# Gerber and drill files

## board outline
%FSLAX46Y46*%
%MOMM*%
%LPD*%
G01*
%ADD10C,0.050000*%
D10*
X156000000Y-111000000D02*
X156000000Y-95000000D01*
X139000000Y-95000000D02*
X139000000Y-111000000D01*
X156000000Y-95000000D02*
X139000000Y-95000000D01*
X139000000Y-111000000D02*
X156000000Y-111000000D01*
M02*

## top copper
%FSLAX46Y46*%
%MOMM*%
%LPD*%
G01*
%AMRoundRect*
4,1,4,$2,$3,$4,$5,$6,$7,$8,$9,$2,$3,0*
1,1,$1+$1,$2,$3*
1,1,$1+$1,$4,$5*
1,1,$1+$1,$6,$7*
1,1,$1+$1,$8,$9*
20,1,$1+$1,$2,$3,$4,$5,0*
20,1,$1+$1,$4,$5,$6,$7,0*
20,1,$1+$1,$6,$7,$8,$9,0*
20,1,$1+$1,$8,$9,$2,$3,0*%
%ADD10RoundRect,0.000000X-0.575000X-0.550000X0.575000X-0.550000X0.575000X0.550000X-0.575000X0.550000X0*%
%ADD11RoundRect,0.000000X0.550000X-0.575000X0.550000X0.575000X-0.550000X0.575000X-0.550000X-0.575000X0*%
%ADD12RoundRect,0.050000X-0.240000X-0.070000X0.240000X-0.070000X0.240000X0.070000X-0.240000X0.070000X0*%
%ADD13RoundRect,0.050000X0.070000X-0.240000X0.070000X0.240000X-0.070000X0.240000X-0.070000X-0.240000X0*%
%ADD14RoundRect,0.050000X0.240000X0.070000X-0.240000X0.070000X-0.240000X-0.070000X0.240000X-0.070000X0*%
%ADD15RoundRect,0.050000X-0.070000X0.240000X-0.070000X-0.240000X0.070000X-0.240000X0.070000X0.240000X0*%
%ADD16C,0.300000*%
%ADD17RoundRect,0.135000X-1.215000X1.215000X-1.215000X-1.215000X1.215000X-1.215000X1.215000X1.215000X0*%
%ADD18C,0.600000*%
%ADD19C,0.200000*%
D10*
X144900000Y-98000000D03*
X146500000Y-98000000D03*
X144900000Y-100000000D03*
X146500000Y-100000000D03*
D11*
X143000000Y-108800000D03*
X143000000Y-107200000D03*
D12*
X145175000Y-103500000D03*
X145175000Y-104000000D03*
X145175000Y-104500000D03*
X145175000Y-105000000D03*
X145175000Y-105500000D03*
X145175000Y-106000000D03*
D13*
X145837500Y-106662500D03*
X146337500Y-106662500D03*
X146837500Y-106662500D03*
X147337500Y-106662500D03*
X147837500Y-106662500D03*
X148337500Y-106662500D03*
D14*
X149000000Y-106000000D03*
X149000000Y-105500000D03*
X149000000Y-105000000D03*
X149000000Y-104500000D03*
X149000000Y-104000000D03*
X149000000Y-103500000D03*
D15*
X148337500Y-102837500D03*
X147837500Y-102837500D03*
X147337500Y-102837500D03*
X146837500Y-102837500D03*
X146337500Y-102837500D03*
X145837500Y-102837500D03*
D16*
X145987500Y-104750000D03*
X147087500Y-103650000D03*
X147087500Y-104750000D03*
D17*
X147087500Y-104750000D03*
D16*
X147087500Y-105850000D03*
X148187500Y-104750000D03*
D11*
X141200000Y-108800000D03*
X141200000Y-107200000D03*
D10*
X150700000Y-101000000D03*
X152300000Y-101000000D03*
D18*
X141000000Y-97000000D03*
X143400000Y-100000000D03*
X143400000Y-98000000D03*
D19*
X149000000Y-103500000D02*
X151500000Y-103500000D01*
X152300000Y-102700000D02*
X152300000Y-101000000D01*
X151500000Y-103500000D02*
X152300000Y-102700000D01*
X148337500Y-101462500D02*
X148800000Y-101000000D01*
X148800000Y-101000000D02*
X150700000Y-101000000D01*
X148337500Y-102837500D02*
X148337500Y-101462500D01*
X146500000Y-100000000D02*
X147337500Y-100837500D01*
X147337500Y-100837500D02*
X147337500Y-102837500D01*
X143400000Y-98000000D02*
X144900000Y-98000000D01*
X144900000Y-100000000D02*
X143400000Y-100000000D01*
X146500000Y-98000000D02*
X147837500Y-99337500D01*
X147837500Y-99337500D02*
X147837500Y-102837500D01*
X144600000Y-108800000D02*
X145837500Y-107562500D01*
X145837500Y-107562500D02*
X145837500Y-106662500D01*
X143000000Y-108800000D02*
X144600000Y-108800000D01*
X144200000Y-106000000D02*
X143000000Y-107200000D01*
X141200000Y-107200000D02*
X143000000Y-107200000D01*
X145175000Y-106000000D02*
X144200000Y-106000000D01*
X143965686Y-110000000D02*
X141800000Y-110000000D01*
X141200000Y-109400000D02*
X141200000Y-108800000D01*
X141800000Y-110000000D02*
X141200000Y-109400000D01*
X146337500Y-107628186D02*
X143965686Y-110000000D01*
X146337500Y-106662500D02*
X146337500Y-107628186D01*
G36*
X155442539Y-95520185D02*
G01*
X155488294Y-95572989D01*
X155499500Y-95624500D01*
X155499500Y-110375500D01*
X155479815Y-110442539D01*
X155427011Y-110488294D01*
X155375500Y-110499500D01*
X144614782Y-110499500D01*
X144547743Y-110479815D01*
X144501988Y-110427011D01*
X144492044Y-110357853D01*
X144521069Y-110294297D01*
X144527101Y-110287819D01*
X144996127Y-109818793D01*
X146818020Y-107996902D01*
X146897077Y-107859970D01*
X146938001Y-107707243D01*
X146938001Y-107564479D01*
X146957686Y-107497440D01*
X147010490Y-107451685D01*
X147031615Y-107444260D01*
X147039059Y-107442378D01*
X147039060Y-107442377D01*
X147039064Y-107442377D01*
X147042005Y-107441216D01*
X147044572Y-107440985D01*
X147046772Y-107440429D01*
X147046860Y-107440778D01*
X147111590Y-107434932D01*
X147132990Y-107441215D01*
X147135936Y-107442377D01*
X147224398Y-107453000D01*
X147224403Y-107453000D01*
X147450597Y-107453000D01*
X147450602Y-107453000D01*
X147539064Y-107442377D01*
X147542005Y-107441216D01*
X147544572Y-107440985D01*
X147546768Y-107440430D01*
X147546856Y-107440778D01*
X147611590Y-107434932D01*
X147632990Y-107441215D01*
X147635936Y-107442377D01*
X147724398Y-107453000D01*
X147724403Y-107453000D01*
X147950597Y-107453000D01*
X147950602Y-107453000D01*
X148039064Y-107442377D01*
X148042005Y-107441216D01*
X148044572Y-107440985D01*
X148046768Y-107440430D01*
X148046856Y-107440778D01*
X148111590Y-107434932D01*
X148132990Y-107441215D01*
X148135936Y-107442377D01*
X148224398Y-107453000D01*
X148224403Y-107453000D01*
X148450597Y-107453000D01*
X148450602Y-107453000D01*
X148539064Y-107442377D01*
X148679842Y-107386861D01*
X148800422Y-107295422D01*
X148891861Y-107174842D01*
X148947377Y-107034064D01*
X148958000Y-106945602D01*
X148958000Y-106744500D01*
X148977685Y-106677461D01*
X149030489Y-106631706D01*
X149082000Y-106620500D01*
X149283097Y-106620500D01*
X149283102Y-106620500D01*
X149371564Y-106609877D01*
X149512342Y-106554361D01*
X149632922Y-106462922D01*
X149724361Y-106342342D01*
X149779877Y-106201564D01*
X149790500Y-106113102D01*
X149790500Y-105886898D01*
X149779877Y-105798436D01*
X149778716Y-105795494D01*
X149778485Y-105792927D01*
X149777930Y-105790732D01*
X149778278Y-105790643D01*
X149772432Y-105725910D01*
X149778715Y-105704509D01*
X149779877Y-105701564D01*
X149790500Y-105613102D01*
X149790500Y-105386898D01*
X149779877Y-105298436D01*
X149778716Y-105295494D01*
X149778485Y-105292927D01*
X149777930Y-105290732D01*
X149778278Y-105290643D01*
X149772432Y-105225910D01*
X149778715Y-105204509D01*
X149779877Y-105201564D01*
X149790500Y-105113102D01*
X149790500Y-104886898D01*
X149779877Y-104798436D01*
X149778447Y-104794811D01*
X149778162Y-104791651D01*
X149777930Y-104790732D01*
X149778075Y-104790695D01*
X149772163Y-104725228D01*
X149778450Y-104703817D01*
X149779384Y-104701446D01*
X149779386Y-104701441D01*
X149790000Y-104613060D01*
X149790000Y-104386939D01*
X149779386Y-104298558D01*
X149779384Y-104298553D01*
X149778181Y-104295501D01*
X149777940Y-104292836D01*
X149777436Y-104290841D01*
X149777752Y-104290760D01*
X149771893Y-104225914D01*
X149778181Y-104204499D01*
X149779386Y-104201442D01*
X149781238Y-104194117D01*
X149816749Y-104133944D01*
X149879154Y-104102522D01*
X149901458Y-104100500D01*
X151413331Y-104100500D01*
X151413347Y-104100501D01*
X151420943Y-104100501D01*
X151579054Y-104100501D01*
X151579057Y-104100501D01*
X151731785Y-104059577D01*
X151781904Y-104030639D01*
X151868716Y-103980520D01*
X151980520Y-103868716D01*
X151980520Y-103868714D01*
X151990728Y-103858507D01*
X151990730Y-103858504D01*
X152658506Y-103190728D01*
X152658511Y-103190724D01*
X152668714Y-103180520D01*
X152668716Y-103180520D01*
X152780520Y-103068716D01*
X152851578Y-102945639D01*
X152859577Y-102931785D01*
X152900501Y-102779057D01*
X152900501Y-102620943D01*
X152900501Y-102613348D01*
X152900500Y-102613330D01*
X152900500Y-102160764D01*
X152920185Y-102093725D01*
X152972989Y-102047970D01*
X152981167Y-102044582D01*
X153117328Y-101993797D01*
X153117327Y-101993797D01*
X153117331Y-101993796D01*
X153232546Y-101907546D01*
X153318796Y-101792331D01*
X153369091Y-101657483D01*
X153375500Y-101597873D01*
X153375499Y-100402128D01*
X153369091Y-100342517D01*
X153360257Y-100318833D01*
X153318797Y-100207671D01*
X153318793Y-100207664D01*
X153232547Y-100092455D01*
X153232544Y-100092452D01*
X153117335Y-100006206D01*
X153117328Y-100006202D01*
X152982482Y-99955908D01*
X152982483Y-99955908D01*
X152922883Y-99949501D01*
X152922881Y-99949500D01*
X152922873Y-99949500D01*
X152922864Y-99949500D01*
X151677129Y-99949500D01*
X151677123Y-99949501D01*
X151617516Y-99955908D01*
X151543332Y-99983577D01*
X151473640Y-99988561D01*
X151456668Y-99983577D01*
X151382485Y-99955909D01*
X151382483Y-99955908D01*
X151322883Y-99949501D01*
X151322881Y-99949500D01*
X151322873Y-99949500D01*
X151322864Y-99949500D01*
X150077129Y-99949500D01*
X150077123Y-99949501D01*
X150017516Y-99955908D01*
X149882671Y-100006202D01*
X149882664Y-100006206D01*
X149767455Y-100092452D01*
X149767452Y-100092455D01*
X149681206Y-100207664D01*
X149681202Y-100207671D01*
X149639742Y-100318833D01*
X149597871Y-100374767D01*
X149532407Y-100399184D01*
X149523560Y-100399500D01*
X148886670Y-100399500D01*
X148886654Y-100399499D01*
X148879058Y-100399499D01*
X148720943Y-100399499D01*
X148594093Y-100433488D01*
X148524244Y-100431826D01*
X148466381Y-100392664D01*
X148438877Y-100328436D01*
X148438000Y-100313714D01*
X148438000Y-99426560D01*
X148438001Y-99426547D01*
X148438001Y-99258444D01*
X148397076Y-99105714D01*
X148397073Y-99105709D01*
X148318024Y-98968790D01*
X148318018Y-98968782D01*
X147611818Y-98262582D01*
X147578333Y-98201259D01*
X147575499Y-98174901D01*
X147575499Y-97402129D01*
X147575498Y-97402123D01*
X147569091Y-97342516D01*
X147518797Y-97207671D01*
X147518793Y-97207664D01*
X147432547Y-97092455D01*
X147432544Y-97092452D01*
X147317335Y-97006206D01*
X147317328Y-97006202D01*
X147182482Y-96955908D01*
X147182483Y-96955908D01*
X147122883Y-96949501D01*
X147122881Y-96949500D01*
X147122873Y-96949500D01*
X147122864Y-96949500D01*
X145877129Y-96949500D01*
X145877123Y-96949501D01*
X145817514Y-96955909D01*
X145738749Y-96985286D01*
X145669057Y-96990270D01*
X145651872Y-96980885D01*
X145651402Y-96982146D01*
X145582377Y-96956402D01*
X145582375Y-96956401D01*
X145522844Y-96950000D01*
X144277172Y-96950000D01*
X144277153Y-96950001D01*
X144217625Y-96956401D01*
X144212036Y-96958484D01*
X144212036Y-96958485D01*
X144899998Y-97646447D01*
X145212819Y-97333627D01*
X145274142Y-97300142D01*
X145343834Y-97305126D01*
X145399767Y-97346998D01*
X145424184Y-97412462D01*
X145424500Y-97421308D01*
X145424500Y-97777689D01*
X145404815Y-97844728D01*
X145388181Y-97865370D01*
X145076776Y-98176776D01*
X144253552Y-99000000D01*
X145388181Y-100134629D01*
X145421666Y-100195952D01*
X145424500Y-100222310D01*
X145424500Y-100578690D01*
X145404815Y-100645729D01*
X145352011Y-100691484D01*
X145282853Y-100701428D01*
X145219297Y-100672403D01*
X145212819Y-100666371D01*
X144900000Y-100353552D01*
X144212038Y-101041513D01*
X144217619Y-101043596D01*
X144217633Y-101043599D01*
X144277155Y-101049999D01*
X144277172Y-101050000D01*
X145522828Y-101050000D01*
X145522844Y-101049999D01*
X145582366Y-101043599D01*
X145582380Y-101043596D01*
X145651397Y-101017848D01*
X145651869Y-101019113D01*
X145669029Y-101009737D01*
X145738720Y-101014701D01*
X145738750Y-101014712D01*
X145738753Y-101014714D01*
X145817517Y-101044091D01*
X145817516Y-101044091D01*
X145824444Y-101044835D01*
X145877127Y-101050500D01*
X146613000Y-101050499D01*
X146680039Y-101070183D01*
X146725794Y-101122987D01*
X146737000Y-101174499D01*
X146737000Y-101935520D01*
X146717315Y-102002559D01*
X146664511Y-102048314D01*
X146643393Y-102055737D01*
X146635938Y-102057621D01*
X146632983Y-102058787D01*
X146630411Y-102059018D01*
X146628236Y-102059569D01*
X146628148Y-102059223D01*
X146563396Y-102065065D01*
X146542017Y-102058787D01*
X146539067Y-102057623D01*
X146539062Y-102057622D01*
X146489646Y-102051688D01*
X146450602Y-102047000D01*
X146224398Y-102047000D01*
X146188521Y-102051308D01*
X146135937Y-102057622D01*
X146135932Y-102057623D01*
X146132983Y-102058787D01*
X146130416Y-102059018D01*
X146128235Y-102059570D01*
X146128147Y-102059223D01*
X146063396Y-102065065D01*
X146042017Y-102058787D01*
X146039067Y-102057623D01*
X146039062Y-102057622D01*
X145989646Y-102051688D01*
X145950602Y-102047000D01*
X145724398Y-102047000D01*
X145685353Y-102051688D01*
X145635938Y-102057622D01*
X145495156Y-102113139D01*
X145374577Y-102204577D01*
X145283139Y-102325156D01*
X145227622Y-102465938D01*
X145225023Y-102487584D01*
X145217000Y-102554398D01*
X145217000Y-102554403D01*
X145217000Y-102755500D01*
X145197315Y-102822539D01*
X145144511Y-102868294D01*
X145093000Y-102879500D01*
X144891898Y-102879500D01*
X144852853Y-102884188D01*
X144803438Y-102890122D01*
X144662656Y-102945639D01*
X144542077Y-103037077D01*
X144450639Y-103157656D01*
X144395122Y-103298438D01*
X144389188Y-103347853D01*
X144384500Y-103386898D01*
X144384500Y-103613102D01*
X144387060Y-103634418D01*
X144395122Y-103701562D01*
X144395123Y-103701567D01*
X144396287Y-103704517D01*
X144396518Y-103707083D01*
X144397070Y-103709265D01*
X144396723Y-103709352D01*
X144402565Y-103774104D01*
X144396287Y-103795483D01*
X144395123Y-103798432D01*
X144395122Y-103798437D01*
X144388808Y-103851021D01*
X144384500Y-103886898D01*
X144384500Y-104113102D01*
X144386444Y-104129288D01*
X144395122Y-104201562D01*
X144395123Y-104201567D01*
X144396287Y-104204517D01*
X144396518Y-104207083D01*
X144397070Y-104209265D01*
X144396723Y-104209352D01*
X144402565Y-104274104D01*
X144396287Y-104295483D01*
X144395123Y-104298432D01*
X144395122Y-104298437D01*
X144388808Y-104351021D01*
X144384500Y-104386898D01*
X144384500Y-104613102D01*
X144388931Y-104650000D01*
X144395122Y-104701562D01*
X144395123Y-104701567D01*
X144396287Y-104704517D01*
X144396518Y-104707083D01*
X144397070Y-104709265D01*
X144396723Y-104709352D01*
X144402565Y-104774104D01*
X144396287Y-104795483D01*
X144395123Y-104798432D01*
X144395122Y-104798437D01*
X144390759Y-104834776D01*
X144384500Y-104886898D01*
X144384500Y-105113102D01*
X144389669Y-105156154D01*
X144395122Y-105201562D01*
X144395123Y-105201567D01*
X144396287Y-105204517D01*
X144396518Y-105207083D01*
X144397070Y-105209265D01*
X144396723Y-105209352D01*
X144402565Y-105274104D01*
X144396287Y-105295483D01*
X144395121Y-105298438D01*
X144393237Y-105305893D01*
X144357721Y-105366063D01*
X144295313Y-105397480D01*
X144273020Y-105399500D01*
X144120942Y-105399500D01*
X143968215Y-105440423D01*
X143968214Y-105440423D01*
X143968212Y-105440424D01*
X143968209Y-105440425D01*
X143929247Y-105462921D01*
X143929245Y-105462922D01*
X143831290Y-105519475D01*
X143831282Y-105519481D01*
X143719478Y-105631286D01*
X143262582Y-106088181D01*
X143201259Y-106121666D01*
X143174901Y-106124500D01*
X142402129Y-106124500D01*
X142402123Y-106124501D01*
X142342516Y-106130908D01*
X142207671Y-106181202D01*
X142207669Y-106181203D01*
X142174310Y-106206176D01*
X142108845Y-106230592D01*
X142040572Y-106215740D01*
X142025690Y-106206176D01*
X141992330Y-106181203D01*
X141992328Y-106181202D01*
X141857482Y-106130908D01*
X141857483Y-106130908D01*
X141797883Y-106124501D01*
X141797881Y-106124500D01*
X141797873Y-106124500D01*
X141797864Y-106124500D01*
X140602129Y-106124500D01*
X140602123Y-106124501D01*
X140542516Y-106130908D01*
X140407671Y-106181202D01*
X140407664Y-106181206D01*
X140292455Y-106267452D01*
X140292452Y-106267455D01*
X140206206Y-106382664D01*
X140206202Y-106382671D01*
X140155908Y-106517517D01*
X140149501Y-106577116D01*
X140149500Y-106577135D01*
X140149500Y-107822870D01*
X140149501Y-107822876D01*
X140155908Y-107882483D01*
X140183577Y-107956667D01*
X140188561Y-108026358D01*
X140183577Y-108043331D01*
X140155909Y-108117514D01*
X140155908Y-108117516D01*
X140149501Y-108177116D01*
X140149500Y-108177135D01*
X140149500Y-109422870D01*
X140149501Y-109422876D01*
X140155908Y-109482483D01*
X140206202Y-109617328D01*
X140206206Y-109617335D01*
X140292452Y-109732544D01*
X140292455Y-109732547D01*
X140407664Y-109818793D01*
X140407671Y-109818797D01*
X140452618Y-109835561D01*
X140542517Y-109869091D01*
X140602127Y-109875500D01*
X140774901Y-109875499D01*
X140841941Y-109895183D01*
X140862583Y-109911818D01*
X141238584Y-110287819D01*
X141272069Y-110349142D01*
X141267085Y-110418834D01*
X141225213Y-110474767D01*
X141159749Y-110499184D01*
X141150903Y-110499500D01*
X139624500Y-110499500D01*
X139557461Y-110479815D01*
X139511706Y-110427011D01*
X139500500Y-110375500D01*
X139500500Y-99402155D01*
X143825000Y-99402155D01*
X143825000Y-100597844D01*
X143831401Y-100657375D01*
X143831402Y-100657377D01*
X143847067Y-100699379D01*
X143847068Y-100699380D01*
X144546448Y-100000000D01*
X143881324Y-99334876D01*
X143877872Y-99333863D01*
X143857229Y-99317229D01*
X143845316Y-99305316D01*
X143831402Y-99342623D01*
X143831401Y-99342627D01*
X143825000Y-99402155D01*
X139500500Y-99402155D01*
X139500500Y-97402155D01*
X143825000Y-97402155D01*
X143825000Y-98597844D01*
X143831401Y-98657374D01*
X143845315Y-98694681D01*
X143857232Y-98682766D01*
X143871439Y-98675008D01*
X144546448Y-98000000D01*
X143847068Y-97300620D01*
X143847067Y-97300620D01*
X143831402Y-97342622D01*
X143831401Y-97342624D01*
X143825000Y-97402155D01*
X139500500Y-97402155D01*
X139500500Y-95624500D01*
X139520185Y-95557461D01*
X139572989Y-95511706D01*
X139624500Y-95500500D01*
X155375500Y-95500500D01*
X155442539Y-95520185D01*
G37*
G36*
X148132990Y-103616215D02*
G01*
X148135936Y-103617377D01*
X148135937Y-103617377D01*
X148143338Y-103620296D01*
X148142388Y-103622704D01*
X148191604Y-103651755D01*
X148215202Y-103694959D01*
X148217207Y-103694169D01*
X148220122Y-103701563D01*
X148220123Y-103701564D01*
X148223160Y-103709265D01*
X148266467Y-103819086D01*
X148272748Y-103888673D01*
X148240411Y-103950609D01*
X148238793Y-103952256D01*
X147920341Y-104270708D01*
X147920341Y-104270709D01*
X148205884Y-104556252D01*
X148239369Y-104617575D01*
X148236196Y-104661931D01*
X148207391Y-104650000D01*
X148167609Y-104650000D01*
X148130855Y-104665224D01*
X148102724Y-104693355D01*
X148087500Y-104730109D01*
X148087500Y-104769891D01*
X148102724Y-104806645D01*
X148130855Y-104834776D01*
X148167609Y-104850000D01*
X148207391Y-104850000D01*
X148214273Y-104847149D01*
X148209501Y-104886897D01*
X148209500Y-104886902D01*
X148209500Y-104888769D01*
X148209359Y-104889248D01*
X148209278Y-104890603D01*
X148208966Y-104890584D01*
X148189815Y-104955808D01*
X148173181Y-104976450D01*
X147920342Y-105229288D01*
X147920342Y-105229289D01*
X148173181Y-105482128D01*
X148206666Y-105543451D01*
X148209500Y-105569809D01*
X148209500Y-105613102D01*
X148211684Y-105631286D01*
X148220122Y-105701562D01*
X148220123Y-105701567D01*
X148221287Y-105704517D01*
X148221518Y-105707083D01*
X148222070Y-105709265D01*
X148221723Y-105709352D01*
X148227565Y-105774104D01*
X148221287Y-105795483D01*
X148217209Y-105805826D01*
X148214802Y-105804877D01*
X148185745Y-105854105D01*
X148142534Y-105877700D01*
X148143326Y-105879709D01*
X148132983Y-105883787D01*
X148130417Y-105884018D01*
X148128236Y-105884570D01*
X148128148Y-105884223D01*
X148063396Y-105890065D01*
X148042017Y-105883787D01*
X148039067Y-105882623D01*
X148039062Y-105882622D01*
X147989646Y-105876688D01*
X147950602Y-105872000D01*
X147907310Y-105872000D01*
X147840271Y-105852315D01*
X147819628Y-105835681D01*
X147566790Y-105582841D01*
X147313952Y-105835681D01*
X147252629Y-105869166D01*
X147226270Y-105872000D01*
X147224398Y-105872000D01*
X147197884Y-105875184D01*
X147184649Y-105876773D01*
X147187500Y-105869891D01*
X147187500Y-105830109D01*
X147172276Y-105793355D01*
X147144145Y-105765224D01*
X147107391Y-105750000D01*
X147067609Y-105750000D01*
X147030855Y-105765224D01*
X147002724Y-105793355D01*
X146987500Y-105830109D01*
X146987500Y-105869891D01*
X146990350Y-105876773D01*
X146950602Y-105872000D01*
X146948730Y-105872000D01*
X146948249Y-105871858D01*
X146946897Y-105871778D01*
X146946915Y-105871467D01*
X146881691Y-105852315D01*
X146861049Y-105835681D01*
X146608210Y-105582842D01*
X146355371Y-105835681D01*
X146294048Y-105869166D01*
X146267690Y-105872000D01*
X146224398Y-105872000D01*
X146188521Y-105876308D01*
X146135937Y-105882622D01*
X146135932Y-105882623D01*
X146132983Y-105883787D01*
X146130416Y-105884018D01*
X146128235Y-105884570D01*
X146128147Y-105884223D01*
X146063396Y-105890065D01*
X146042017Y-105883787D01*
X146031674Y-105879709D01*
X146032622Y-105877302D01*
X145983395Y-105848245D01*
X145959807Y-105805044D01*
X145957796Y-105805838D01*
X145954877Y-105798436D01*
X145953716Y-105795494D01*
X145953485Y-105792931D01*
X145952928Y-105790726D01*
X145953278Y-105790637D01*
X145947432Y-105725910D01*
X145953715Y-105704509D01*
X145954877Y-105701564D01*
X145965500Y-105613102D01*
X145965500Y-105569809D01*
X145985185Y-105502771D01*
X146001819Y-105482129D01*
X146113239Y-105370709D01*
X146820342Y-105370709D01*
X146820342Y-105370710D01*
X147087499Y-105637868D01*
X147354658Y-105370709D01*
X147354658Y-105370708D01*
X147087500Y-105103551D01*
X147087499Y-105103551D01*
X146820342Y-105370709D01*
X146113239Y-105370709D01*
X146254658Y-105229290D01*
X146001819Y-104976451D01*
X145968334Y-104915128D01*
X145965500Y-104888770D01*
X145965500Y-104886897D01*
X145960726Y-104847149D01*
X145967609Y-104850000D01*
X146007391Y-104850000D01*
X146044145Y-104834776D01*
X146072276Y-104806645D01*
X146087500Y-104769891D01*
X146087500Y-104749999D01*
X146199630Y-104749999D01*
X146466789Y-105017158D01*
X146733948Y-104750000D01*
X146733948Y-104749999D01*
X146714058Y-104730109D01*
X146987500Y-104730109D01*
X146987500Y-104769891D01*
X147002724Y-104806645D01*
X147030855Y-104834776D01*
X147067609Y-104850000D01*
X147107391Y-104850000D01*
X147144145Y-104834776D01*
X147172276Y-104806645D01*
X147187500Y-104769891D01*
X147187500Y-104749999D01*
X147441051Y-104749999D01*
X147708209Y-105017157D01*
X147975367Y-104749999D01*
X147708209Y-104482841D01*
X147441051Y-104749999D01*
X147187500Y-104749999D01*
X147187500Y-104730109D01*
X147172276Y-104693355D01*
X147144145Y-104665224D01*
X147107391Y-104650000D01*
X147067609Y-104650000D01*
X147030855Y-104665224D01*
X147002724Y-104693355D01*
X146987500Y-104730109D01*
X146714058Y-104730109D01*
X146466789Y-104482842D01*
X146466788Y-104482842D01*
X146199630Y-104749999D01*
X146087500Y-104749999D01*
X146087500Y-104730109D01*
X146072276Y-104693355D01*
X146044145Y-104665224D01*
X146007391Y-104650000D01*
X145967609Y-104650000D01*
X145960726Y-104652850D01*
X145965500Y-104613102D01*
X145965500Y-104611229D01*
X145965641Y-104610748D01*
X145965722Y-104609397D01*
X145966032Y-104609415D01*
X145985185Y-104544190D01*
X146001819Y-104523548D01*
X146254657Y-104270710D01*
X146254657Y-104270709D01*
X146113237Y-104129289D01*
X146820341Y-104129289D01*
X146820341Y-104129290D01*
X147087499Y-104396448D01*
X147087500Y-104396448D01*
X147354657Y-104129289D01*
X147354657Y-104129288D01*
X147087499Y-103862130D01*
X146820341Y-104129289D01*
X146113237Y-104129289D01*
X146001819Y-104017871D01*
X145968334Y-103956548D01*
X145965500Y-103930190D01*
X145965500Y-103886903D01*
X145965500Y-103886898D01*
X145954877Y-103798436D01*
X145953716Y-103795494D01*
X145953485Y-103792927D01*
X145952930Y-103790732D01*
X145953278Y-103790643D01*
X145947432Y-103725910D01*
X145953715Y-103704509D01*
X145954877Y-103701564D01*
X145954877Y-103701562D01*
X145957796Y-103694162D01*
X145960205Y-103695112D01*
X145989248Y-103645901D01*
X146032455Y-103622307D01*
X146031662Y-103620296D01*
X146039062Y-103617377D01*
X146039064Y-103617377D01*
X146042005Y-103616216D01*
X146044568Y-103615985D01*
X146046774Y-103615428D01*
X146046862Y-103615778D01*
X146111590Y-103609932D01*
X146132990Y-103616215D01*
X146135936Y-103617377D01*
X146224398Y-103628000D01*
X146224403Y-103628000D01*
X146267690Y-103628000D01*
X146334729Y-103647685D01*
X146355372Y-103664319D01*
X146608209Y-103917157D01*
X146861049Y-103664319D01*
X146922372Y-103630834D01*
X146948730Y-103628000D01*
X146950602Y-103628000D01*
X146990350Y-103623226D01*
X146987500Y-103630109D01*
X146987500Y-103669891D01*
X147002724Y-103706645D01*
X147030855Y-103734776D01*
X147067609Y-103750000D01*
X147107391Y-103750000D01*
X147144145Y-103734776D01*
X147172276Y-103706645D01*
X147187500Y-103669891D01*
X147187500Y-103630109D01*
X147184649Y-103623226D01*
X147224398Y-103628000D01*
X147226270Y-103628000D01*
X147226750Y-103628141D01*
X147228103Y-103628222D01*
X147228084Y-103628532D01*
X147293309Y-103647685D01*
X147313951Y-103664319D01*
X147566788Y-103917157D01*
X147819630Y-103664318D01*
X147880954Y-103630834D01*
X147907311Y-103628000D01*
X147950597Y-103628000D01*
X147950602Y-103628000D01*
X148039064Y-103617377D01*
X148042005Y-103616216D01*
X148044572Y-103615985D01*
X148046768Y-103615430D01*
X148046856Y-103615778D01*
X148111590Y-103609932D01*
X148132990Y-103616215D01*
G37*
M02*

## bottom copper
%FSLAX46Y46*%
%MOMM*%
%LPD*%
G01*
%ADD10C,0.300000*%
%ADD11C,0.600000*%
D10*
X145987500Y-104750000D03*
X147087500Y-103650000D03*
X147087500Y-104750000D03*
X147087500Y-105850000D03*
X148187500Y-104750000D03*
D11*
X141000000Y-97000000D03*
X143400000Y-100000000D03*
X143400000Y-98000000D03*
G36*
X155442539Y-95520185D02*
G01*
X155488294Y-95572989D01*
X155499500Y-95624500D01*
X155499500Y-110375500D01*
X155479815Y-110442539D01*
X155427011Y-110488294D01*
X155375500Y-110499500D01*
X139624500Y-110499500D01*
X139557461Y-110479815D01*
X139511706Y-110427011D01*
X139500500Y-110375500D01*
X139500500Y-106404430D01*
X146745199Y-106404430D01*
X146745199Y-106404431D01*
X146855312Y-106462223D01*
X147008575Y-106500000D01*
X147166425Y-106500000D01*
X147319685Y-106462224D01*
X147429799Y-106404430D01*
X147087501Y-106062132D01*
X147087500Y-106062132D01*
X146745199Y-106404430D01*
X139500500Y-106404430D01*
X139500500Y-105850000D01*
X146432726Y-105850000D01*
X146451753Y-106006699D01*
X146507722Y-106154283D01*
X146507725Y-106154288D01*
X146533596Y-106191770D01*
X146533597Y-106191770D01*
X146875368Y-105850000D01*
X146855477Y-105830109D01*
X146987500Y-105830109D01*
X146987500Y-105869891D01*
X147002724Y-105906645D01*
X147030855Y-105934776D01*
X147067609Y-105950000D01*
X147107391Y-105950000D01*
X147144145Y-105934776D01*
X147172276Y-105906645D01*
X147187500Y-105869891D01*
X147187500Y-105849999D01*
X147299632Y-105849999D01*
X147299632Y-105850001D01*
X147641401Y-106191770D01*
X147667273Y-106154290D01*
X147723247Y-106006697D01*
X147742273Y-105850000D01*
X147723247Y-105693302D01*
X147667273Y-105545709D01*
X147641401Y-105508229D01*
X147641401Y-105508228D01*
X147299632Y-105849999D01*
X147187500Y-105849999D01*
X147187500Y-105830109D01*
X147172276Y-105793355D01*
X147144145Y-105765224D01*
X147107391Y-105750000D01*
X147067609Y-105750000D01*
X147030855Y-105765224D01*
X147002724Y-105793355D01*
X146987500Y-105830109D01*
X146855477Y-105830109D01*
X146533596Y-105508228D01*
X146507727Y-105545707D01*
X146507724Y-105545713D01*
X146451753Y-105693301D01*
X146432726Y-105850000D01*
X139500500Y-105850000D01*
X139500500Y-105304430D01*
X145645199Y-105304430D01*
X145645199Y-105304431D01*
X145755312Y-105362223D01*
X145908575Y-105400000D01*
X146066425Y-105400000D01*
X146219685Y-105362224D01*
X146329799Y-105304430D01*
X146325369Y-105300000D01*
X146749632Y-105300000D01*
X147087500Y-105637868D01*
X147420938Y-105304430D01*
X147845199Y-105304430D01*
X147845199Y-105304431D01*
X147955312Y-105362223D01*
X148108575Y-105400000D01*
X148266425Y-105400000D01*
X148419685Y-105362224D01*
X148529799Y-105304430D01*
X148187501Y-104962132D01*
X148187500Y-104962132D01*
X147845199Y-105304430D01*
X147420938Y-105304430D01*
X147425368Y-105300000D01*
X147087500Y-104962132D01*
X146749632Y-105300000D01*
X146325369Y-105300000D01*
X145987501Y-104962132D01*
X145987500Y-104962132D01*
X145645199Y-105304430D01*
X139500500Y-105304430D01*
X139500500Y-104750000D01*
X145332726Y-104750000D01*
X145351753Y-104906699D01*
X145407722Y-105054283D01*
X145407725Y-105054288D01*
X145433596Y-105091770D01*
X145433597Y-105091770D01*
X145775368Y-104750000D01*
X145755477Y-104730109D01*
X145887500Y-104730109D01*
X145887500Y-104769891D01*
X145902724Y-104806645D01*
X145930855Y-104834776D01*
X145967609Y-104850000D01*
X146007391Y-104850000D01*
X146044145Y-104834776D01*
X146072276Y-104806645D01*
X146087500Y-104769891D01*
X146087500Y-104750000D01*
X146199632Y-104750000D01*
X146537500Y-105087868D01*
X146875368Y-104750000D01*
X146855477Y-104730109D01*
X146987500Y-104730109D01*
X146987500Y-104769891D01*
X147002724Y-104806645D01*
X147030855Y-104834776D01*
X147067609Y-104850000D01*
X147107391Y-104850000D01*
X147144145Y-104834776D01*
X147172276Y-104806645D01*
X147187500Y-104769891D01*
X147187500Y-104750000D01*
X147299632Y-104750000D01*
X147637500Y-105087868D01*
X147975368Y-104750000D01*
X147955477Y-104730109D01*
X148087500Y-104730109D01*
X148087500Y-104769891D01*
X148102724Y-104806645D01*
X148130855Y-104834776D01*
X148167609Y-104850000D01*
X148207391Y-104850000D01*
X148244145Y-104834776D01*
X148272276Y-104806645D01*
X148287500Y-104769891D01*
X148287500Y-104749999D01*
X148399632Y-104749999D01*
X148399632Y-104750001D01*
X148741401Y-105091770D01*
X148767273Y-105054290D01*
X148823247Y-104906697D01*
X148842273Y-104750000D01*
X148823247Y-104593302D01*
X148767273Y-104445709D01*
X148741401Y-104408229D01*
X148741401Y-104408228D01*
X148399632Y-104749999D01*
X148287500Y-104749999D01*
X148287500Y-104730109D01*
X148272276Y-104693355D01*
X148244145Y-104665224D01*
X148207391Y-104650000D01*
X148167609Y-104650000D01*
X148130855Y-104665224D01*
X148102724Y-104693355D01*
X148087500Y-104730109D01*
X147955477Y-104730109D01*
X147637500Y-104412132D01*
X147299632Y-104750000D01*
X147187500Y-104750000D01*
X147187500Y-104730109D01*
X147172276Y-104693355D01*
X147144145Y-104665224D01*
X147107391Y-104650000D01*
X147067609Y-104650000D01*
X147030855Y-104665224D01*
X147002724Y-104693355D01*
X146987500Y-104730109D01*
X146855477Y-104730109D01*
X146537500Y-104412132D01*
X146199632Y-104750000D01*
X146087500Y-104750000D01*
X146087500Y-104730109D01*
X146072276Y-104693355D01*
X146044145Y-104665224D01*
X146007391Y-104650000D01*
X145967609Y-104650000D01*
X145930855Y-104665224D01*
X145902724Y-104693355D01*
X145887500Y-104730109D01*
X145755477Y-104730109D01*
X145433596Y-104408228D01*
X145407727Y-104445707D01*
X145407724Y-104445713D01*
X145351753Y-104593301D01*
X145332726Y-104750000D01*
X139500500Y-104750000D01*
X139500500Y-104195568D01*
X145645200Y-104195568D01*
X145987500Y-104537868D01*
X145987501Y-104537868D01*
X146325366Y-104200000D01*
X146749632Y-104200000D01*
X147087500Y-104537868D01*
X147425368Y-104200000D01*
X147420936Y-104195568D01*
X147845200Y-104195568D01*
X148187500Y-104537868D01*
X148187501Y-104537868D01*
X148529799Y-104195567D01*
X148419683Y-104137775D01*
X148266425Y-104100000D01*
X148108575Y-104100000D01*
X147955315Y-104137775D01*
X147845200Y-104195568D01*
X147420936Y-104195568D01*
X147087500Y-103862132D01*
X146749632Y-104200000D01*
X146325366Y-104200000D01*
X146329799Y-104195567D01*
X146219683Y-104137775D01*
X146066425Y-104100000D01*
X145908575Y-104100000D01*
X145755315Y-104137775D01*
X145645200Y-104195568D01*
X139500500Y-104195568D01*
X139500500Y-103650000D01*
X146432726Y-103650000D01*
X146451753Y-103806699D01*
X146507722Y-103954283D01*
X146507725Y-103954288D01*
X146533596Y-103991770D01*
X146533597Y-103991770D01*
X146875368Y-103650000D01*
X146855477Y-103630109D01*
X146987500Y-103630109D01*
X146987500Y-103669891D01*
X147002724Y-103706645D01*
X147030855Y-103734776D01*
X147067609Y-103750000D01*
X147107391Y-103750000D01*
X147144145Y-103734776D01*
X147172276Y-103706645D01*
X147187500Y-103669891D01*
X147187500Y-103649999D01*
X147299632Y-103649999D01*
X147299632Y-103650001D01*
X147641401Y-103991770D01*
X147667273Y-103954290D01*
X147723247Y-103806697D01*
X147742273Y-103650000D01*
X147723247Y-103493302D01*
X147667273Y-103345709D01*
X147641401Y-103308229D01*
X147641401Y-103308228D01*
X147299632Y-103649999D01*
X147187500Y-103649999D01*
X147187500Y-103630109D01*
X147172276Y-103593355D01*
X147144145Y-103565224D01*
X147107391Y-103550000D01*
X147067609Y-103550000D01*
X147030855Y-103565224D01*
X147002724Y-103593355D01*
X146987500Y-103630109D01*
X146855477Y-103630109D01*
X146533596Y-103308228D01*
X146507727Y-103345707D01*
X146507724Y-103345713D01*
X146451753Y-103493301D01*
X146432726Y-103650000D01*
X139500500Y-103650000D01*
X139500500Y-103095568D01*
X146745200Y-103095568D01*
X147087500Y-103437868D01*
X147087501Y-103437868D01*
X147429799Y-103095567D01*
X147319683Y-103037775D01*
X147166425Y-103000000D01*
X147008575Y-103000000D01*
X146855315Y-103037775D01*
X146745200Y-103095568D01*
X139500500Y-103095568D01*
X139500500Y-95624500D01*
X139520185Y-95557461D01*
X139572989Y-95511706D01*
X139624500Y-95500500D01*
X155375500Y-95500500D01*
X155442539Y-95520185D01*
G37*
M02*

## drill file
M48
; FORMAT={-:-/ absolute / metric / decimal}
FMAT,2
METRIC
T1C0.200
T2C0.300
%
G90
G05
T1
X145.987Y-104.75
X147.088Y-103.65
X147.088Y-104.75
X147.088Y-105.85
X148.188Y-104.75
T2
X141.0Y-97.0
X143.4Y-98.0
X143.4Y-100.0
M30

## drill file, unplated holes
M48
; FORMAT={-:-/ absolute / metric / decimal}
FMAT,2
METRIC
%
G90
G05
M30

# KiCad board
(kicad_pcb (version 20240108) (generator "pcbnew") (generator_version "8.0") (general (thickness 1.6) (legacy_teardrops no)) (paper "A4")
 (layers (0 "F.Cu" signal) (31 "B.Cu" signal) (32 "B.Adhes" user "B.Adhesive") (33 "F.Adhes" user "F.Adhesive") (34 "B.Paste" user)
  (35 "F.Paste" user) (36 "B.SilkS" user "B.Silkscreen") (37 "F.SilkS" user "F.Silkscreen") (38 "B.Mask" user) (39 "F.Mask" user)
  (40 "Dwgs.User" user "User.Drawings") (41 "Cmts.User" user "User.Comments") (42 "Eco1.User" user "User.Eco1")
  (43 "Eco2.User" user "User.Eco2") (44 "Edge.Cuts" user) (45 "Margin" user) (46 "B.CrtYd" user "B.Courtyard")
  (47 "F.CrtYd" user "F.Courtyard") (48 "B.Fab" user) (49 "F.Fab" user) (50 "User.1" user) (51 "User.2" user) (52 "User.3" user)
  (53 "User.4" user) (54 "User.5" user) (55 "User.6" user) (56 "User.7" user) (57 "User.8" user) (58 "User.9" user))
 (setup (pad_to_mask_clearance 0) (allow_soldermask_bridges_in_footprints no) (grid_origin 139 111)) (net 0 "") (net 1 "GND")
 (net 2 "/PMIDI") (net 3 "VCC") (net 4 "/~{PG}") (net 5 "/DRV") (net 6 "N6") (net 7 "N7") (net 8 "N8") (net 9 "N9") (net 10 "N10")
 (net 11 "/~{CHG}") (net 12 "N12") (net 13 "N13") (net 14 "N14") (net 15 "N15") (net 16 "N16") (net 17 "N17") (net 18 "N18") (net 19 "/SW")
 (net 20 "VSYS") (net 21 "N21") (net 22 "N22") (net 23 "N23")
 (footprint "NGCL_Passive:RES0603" (layer "F.Cu") (at 145.7 98)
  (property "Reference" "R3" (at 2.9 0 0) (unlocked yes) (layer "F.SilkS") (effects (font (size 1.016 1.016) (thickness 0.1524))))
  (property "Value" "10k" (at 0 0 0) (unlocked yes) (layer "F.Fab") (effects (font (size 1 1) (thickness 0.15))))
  (pad "1" smd roundrect (at -0.8 0) (size 1.15 1.1) (layers "F.Cu" "F.Paste" "F.Mask") (roundrect_rratio 0) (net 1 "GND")
   (thermal_bridge_angle 45))
  (pad "2" smd roundrect (at 0.8 0) (size 1.15 1.1) (layers "F.Cu" "F.Paste" "F.Mask") (roundrect_rratio 0) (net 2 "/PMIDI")
   (thermal_bridge_angle 45)))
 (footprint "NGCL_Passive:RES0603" (layer "F.Cu") (at 145.7 100)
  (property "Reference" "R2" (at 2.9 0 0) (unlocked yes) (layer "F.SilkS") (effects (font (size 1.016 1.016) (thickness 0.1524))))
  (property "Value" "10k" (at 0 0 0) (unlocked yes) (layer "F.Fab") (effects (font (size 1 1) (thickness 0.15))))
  (pad "1" smd roundrect (at -0.8 0) (size 1.15 1.1) (layers "F.Cu" "F.Paste" "F.Mask") (roundrect_rratio 0) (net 1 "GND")
   (thermal_bridge_angle 45))
  (pad "2" smd roundrect (at 0.8 0) (size 1.15 1.1) (layers "F.Cu" "F.Paste" "F.Mask") (roundrect_rratio 0) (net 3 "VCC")
   (thermal_bridge_angle 45)))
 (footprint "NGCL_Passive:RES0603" (layer "F.Cu") (at 143 108 90)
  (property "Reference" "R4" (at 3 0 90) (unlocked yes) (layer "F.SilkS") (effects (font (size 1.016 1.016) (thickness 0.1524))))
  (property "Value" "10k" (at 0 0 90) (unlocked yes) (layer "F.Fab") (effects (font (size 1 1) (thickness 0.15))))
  (pad "1" smd roundrect (at -0.8 0 90) (size 1.15 1.1) (layers "F.Cu" "F.Paste" "F.Mask") (roundrect_rratio 0) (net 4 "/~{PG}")
   (thermal_bridge_angle 45))
  (pad "2" smd roundrect (at 0.8 0 90) (size 1.15 1.1) (layers "F.Cu" "F.Paste" "F.Mask") (roundrect_rratio 0) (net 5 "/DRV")
   (thermal_bridge_angle 45)))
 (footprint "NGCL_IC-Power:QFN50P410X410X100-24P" (layer "F.Cu") (at 147.0875 104.75)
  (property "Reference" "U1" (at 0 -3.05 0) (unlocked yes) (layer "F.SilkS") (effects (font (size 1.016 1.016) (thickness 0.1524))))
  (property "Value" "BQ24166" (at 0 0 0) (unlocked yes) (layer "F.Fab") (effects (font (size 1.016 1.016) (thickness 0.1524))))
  (pad "1" smd roundrect (at -1.9125 -1.25) (size 0.58 0.24) (layers "F.Cu" "F.Paste" "F.Mask") (roundrect_rratio 0.2083333333) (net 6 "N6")
   (solder_mask_margin 0.07) (thermal_bridge_angle 45))
  (pad "2" smd roundrect (at -1.9125 -0.75) (size 0.58 0.24) (layers "F.Cu" "F.Paste" "F.Mask") (roundrect_rratio 0.2083333333) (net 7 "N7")
   (solder_mask_margin 0.07) (thermal_bridge_angle 45))
  (pad "3" smd roundrect (at -1.9125 -0.25) (size 0.58 0.24) (layers "F.Cu" "F.Paste" "F.Mask") (roundrect_rratio 0.2083333333) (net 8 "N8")
   (solder_mask_margin 0.07) (thermal_bridge_angle 45))
  (pad "4" smd roundrect (at -1.9125 0.25) (size 0.58 0.24) (layers "F.Cu" "F.Paste" "F.Mask") (roundrect_rratio 0.2083333333) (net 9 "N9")
   (solder_mask_margin 0.07) (thermal_bridge_angle 45))
  (pad "5" smd roundrect (at -1.9125 0.75) (size 0.58 0.24) (layers "F.Cu" "F.Paste" "F.Mask") (roundrect_rratio 0.2083333333)
   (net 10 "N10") (solder_mask_margin 0.07) (thermal_bridge_angle 45))
  (pad "6" smd roundrect (at -1.9125 1.25) (size 0.58 0.24) (layers "F.Cu" "F.Paste" "F.Mask") (roundrect_rratio 0.2083333333)
   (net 5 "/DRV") (solder_mask_margin 0.07) (thermal_bridge_angle 45))
  (pad "7" smd roundrect (at -1.25 1.9125 90) (size 0.58 0.24) (layers "F.Cu" "F.Paste" "F.Mask") (roundrect_rratio 0.2083333333)
   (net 4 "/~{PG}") (solder_mask_margin 0.07) (thermal_bridge_angle 45))
  (pad "8" smd roundrect (at -0.75 1.9125 90) (size 0.58 0.24) (layers "F.Cu" "F.Paste" "F.Mask") (roundrect_rratio 0.2083333333)
   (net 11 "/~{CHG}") (solder_mask_margin 0.07) (thermal_bridge_angle 45))
  (pad "9" smd roundrect (at -0.25 1.9125 90) (size 0.58 0.24) (layers "F.Cu" "F.Paste" "F.Mask") (roundrect_rratio 0.2083333333)
   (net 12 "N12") (solder_mask_margin 0.07) (thermal_bridge_angle 45))
  (pad "10" smd roundrect (at 0.25 1.9125 90) (size 0.58 0.24) (layers "F.Cu" "F.Paste" "F.Mask") (roundrect_rratio 0.2083333333)
   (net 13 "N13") (solder_mask_margin 0.07) (thermal_bridge_angle 45))
  (pad "11" smd roundrect (at 0.75 1.9125 90) (size 0.58 0.24) (layers "F.Cu" "F.Paste" "F.Mask") (roundrect_rratio 0.2083333333)
   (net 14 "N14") (solder_mask_margin 0.07) (thermal_bridge_angle 45))
  (pad "12" smd roundrect (at 1.25 1.9125 90) (size 0.58 0.24) (layers "F.Cu" "F.Paste" "F.Mask") (roundrect_rratio 0.2083333333)
   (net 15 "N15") (solder_mask_margin 0.07) (thermal_bridge_angle 45))
  (pad "13" smd roundrect (at 1.9125 1.25 180) (size 0.58 0.24) (layers "F.Cu" "F.Paste" "F.Mask") (roundrect_rratio 0.2083333333)
   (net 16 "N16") (solder_mask_margin 0.07) (thermal_bridge_angle 45))
  (pad "14" smd roundrect (at 1.9125 0.75 180) (size 0.58 0.24) (layers "F.Cu" "F.Paste" "F.Mask") (roundrect_rratio 0.2083333333)
   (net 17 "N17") (solder_mask_margin 0.07) (thermal_bridge_angle 45))
  (pad "15" smd roundrect (at 1.9125 0.25 180) (size 0.58 0.24) (layers "F.Cu" "F.Paste" "F.Mask") (roundrect_rratio 0.2083333333)
   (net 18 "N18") (solder_mask_margin 0.07) (thermal_bridge_angle 45))
  (pad "16" smd roundrect (at 1.9125 -0.25 180) (size 0.58 0.24) (layers "F.Cu" "F.Paste" "F.Mask") (roundrect_rratio 0.2083333333)
   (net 1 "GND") (solder_mask_margin 0.07) (thermal_bridge_angle 45))
  (pad "17" smd roundrect (at 1.9125 -0.75 180) (size 0.58 0.24) (layers "F.Cu" "F.Paste" "F.Mask") (roundrect_rratio 0.2083333333)
   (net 1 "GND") (solder_mask_margin 0.07) (thermal_bridge_angle 45))
  (pad "18" smd roundrect (at 1.9125 -1.25 180) (size 0.58 0.24) (layers "F.Cu" "F.Paste" "F.Mask") (roundrect_rratio 0.2083333333)
   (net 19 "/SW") (solder_mask_margin 0.07) (thermal_bridge_angle 45))
  (pad "19" smd roundrect (at 1.25 -1.9125 270) (size 0.58 0.24) (layers "F.Cu" "F.Paste" "F.Mask") (roundrect_rratio 0.2083333333)
   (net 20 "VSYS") (solder_mask_margin 0.07) (thermal_bridge_angle 45))
  (pad "20" smd roundrect (at 0.75 -1.9125 270) (size 0.58 0.24) (layers "F.Cu" "F.Paste" "F.Mask") (roundrect_rratio 0.2083333333)
   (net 2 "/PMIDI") (solder_mask_margin 0.07) (thermal_bridge_angle 45))
  (pad "21" smd roundrect (at 0.25 -1.9125 270) (size 0.58 0.24) (layers "F.Cu" "F.Paste" "F.Mask") (roundrect_rratio 0.2083333333)
   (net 3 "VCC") (solder_mask_margin 0.07) (thermal_bridge_angle 45))
  (pad "22" smd roundrect (at -0.25 -1.9125 270) (size 0.58 0.24) (layers "F.Cu" "F.Paste" "F.Mask") (roundrect_rratio 0.2083333333)
   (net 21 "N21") (solder_mask_margin 0.07) (thermal_bridge_angle 45))
  (pad "23" smd roundrect (at -0.75 -1.9125 270) (size 0.58 0.24) (layers "F.Cu" "F.Paste" "F.Mask") (roundrect_rratio 0.2083333333)
   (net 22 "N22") (solder_mask_margin 0.07) (thermal_bridge_angle 45))
  (pad "24" smd roundrect (at -1.25 -1.9125 270) (size 0.58 0.24) (layers "F.Cu" "F.Paste" "F.Mask") (roundrect_rratio 0.2083333333)
   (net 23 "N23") (solder_mask_margin 0.07) (thermal_bridge_angle 45))
  (pad "25" thru_hole circle (at -1.1 0) (size 0.3 0.3) (drill 0.2) (layers "*.Cu") (remove_unused_layers no) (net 1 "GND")
   (solder_mask_margin 0.07))
  (pad "25" thru_hole circle (at 0 -1.1) (size 0.3 0.3) (drill 0.2) (layers "*.Cu") (remove_unused_layers no) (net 1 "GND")
   (solder_mask_margin 0.07))
  (pad "25" thru_hole circle (at 0 0) (size 0.3 0.3) (drill 0.2) (layers "*.Cu") (remove_unused_layers no) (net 1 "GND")
   (solder_mask_margin 0.07))
  (pad "25" smd roundrect (at 0 0 270) (size 2.7 2.7) (layers "F.Cu" "F.Paste" "F.Mask") (roundrect_rratio 0.05) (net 1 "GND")
   (solder_mask_margin 0.07) (thermal_bridge_angle 45))
  (pad "25" thru_hole circle (at 0 1.1) (size 0.3 0.3) (drill 0.2) (layers "*.Cu") (remove_unused_layers no) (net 1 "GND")
   (solder_mask_margin 0.07))
  (pad "25" thru_hole circle (at 1.1 0) (size 0.3 0.3) (drill 0.2) (layers "*.Cu") (remove_unused_layers no) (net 1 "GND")
   (solder_mask_margin 0.07)))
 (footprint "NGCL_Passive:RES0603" (layer "F.Cu") (at 141.2 108 90)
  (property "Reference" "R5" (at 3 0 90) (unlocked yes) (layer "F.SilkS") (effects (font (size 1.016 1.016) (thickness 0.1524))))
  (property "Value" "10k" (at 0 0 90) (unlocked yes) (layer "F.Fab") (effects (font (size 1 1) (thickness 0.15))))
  (pad "1" smd roundrect (at -0.8 0 90) (size 1.15 1.1) (layers "F.Cu" "F.Paste" "F.Mask") (roundrect_rratio 0) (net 11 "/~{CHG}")
   (thermal_bridge_angle 45))
  (pad "2" smd roundrect (at 0.8 0 90) (size 1.15 1.1) (layers "F.Cu" "F.Paste" "F.Mask") (roundrect_rratio 0) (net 5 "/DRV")
   (thermal_bridge_angle 45)))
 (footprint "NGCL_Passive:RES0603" (layer "F.Cu") (at 151.5 101)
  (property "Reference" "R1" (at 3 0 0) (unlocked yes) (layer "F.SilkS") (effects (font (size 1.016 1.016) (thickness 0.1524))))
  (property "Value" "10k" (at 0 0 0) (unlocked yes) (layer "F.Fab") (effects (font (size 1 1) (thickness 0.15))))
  (pad "1" smd roundrect (at -0.8 0) (size 1.15 1.1) (layers "F.Cu" "F.Paste" "F.Mask") (roundrect_rratio 0) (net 20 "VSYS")
   (thermal_bridge_angle 45))
  (pad "2" smd roundrect (at 0.8 0) (size 1.15 1.1) (layers "F.Cu" "F.Paste" "F.Mask") (roundrect_rratio 0) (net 19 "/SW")
   (thermal_bridge_angle 45)))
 (gr_line (start 156 111) (end 156 95) (stroke (width 0.05) (type default)) (layer "Edge.Cuts"))
 (gr_line (start 139 95) (end 139 111) (stroke (width 0.05) (type default)) (layer "Edge.Cuts"))
 (gr_line (start 156 95) (end 139 95) (stroke (width 0.05) (type default)) (layer "Edge.Cuts"))
 (gr_line (start 139 111) (end 156 111) (stroke (width 0.05) (type default)) (layer "Edge.Cuts"))
 (segment (start 149 103.5) (end 151.5 103.5) (width 0.2) (layer "F.Cu") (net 19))
 (segment (start 152.3 102.7) (end 152.3 101) (width 0.2) (layer "F.Cu") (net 19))
 (segment (start 151.5 103.5) (end 152.3 102.7) (width 0.2) (layer "F.Cu") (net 19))
 (segment (start 148.3375 101.4625) (end 148.8 101) (width 0.2) (layer "F.Cu") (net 20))
 (segment (start 148.8 101) (end 150.7 101) (width 0.2) (layer "F.Cu") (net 20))
 (segment (start 148.3375 102.8375) (end 148.3375 101.4625) (width 0.2) (layer "F.Cu") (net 20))
 (segment (start 146.5 100) (end 147.3375 100.8375) (width 0.2) (layer "F.Cu") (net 3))
 (segment (start 147.3375 100.8375) (end 147.3375 102.8375) (width 0.2) (layer "F.Cu") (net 3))
 (segment (start 143.4 98) (end 144.9 98) (width 0.2) (layer "F.Cu") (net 1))
 (segment (start 144.9 100) (end 143.4 100) (width 0.2) (layer "F.Cu") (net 1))
 (via (at 141 97) (size 0.6) (drill 0.3) (layers "F.Cu" "B.Cu") (free yes) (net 1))
 (via (at 143.4 100) (size 0.6) (drill 0.3) (layers "F.Cu" "B.Cu") (free yes) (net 1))
 (via (at 143.4 98) (size 0.6) (drill 0.3) (layers "F.Cu" "B.Cu") (free yes) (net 1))
 (segment (start 146.5 98) (end 147.8375 99.3375) (width 0.2) (layer "F.Cu") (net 2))
 (segment (start 147.8375 99.3375) (end 147.8375 102.8375) (width 0.2) (layer "F.Cu") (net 2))
 (segment (start 144.6 108.8) (end 145.8375 107.5625) (width 0.2) (layer "F.Cu") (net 4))
 (segment (start 145.8375 107.5625) (end 145.8375 106.6625) (width 0.2) (layer "F.Cu") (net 4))
 (segment (start 143 108.8) (end 144.6 108.8) (width 0.2) (layer "F.Cu") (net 4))
 (segment (start 144.2 106) (end 143 107.2) (width 0.2) (layer "F.Cu") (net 5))
 (segment (start 141.2 107.2) (end 143 107.2) (width 0.2) (layer "F.Cu") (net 5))
 (segment (start 145.175 106) (end 144.2 106) (width 0.2) (layer "F.Cu") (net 5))
 (segment (start 143.965686 110) (end 141.8 110) (width 0.2) (layer "F.Cu") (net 11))
 (segment (start 141.2 109.4) (end 141.2 108.8) (width 0.2) (layer "F.Cu") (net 11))
 (segment (start 141.8 110) (end 141.2 109.4) (width 0.2) (layer "F.Cu") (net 11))
 (segment (start 146.3375 107.628186) (end 143.965686 110) (width 0.2) (layer "F.Cu") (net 11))
 (segment (start 146.3375 106.6625) (end 146.3375 107.628186) (width 0.2) (layer "F.Cu") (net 11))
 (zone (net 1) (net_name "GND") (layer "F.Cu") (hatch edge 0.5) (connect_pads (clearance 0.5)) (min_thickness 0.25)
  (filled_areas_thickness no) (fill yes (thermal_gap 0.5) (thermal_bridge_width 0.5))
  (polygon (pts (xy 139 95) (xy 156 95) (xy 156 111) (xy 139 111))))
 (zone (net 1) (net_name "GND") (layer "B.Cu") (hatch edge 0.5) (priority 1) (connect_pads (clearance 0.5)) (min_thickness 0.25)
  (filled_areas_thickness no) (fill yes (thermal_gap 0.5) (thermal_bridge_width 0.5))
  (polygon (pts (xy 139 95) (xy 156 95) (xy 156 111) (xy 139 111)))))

